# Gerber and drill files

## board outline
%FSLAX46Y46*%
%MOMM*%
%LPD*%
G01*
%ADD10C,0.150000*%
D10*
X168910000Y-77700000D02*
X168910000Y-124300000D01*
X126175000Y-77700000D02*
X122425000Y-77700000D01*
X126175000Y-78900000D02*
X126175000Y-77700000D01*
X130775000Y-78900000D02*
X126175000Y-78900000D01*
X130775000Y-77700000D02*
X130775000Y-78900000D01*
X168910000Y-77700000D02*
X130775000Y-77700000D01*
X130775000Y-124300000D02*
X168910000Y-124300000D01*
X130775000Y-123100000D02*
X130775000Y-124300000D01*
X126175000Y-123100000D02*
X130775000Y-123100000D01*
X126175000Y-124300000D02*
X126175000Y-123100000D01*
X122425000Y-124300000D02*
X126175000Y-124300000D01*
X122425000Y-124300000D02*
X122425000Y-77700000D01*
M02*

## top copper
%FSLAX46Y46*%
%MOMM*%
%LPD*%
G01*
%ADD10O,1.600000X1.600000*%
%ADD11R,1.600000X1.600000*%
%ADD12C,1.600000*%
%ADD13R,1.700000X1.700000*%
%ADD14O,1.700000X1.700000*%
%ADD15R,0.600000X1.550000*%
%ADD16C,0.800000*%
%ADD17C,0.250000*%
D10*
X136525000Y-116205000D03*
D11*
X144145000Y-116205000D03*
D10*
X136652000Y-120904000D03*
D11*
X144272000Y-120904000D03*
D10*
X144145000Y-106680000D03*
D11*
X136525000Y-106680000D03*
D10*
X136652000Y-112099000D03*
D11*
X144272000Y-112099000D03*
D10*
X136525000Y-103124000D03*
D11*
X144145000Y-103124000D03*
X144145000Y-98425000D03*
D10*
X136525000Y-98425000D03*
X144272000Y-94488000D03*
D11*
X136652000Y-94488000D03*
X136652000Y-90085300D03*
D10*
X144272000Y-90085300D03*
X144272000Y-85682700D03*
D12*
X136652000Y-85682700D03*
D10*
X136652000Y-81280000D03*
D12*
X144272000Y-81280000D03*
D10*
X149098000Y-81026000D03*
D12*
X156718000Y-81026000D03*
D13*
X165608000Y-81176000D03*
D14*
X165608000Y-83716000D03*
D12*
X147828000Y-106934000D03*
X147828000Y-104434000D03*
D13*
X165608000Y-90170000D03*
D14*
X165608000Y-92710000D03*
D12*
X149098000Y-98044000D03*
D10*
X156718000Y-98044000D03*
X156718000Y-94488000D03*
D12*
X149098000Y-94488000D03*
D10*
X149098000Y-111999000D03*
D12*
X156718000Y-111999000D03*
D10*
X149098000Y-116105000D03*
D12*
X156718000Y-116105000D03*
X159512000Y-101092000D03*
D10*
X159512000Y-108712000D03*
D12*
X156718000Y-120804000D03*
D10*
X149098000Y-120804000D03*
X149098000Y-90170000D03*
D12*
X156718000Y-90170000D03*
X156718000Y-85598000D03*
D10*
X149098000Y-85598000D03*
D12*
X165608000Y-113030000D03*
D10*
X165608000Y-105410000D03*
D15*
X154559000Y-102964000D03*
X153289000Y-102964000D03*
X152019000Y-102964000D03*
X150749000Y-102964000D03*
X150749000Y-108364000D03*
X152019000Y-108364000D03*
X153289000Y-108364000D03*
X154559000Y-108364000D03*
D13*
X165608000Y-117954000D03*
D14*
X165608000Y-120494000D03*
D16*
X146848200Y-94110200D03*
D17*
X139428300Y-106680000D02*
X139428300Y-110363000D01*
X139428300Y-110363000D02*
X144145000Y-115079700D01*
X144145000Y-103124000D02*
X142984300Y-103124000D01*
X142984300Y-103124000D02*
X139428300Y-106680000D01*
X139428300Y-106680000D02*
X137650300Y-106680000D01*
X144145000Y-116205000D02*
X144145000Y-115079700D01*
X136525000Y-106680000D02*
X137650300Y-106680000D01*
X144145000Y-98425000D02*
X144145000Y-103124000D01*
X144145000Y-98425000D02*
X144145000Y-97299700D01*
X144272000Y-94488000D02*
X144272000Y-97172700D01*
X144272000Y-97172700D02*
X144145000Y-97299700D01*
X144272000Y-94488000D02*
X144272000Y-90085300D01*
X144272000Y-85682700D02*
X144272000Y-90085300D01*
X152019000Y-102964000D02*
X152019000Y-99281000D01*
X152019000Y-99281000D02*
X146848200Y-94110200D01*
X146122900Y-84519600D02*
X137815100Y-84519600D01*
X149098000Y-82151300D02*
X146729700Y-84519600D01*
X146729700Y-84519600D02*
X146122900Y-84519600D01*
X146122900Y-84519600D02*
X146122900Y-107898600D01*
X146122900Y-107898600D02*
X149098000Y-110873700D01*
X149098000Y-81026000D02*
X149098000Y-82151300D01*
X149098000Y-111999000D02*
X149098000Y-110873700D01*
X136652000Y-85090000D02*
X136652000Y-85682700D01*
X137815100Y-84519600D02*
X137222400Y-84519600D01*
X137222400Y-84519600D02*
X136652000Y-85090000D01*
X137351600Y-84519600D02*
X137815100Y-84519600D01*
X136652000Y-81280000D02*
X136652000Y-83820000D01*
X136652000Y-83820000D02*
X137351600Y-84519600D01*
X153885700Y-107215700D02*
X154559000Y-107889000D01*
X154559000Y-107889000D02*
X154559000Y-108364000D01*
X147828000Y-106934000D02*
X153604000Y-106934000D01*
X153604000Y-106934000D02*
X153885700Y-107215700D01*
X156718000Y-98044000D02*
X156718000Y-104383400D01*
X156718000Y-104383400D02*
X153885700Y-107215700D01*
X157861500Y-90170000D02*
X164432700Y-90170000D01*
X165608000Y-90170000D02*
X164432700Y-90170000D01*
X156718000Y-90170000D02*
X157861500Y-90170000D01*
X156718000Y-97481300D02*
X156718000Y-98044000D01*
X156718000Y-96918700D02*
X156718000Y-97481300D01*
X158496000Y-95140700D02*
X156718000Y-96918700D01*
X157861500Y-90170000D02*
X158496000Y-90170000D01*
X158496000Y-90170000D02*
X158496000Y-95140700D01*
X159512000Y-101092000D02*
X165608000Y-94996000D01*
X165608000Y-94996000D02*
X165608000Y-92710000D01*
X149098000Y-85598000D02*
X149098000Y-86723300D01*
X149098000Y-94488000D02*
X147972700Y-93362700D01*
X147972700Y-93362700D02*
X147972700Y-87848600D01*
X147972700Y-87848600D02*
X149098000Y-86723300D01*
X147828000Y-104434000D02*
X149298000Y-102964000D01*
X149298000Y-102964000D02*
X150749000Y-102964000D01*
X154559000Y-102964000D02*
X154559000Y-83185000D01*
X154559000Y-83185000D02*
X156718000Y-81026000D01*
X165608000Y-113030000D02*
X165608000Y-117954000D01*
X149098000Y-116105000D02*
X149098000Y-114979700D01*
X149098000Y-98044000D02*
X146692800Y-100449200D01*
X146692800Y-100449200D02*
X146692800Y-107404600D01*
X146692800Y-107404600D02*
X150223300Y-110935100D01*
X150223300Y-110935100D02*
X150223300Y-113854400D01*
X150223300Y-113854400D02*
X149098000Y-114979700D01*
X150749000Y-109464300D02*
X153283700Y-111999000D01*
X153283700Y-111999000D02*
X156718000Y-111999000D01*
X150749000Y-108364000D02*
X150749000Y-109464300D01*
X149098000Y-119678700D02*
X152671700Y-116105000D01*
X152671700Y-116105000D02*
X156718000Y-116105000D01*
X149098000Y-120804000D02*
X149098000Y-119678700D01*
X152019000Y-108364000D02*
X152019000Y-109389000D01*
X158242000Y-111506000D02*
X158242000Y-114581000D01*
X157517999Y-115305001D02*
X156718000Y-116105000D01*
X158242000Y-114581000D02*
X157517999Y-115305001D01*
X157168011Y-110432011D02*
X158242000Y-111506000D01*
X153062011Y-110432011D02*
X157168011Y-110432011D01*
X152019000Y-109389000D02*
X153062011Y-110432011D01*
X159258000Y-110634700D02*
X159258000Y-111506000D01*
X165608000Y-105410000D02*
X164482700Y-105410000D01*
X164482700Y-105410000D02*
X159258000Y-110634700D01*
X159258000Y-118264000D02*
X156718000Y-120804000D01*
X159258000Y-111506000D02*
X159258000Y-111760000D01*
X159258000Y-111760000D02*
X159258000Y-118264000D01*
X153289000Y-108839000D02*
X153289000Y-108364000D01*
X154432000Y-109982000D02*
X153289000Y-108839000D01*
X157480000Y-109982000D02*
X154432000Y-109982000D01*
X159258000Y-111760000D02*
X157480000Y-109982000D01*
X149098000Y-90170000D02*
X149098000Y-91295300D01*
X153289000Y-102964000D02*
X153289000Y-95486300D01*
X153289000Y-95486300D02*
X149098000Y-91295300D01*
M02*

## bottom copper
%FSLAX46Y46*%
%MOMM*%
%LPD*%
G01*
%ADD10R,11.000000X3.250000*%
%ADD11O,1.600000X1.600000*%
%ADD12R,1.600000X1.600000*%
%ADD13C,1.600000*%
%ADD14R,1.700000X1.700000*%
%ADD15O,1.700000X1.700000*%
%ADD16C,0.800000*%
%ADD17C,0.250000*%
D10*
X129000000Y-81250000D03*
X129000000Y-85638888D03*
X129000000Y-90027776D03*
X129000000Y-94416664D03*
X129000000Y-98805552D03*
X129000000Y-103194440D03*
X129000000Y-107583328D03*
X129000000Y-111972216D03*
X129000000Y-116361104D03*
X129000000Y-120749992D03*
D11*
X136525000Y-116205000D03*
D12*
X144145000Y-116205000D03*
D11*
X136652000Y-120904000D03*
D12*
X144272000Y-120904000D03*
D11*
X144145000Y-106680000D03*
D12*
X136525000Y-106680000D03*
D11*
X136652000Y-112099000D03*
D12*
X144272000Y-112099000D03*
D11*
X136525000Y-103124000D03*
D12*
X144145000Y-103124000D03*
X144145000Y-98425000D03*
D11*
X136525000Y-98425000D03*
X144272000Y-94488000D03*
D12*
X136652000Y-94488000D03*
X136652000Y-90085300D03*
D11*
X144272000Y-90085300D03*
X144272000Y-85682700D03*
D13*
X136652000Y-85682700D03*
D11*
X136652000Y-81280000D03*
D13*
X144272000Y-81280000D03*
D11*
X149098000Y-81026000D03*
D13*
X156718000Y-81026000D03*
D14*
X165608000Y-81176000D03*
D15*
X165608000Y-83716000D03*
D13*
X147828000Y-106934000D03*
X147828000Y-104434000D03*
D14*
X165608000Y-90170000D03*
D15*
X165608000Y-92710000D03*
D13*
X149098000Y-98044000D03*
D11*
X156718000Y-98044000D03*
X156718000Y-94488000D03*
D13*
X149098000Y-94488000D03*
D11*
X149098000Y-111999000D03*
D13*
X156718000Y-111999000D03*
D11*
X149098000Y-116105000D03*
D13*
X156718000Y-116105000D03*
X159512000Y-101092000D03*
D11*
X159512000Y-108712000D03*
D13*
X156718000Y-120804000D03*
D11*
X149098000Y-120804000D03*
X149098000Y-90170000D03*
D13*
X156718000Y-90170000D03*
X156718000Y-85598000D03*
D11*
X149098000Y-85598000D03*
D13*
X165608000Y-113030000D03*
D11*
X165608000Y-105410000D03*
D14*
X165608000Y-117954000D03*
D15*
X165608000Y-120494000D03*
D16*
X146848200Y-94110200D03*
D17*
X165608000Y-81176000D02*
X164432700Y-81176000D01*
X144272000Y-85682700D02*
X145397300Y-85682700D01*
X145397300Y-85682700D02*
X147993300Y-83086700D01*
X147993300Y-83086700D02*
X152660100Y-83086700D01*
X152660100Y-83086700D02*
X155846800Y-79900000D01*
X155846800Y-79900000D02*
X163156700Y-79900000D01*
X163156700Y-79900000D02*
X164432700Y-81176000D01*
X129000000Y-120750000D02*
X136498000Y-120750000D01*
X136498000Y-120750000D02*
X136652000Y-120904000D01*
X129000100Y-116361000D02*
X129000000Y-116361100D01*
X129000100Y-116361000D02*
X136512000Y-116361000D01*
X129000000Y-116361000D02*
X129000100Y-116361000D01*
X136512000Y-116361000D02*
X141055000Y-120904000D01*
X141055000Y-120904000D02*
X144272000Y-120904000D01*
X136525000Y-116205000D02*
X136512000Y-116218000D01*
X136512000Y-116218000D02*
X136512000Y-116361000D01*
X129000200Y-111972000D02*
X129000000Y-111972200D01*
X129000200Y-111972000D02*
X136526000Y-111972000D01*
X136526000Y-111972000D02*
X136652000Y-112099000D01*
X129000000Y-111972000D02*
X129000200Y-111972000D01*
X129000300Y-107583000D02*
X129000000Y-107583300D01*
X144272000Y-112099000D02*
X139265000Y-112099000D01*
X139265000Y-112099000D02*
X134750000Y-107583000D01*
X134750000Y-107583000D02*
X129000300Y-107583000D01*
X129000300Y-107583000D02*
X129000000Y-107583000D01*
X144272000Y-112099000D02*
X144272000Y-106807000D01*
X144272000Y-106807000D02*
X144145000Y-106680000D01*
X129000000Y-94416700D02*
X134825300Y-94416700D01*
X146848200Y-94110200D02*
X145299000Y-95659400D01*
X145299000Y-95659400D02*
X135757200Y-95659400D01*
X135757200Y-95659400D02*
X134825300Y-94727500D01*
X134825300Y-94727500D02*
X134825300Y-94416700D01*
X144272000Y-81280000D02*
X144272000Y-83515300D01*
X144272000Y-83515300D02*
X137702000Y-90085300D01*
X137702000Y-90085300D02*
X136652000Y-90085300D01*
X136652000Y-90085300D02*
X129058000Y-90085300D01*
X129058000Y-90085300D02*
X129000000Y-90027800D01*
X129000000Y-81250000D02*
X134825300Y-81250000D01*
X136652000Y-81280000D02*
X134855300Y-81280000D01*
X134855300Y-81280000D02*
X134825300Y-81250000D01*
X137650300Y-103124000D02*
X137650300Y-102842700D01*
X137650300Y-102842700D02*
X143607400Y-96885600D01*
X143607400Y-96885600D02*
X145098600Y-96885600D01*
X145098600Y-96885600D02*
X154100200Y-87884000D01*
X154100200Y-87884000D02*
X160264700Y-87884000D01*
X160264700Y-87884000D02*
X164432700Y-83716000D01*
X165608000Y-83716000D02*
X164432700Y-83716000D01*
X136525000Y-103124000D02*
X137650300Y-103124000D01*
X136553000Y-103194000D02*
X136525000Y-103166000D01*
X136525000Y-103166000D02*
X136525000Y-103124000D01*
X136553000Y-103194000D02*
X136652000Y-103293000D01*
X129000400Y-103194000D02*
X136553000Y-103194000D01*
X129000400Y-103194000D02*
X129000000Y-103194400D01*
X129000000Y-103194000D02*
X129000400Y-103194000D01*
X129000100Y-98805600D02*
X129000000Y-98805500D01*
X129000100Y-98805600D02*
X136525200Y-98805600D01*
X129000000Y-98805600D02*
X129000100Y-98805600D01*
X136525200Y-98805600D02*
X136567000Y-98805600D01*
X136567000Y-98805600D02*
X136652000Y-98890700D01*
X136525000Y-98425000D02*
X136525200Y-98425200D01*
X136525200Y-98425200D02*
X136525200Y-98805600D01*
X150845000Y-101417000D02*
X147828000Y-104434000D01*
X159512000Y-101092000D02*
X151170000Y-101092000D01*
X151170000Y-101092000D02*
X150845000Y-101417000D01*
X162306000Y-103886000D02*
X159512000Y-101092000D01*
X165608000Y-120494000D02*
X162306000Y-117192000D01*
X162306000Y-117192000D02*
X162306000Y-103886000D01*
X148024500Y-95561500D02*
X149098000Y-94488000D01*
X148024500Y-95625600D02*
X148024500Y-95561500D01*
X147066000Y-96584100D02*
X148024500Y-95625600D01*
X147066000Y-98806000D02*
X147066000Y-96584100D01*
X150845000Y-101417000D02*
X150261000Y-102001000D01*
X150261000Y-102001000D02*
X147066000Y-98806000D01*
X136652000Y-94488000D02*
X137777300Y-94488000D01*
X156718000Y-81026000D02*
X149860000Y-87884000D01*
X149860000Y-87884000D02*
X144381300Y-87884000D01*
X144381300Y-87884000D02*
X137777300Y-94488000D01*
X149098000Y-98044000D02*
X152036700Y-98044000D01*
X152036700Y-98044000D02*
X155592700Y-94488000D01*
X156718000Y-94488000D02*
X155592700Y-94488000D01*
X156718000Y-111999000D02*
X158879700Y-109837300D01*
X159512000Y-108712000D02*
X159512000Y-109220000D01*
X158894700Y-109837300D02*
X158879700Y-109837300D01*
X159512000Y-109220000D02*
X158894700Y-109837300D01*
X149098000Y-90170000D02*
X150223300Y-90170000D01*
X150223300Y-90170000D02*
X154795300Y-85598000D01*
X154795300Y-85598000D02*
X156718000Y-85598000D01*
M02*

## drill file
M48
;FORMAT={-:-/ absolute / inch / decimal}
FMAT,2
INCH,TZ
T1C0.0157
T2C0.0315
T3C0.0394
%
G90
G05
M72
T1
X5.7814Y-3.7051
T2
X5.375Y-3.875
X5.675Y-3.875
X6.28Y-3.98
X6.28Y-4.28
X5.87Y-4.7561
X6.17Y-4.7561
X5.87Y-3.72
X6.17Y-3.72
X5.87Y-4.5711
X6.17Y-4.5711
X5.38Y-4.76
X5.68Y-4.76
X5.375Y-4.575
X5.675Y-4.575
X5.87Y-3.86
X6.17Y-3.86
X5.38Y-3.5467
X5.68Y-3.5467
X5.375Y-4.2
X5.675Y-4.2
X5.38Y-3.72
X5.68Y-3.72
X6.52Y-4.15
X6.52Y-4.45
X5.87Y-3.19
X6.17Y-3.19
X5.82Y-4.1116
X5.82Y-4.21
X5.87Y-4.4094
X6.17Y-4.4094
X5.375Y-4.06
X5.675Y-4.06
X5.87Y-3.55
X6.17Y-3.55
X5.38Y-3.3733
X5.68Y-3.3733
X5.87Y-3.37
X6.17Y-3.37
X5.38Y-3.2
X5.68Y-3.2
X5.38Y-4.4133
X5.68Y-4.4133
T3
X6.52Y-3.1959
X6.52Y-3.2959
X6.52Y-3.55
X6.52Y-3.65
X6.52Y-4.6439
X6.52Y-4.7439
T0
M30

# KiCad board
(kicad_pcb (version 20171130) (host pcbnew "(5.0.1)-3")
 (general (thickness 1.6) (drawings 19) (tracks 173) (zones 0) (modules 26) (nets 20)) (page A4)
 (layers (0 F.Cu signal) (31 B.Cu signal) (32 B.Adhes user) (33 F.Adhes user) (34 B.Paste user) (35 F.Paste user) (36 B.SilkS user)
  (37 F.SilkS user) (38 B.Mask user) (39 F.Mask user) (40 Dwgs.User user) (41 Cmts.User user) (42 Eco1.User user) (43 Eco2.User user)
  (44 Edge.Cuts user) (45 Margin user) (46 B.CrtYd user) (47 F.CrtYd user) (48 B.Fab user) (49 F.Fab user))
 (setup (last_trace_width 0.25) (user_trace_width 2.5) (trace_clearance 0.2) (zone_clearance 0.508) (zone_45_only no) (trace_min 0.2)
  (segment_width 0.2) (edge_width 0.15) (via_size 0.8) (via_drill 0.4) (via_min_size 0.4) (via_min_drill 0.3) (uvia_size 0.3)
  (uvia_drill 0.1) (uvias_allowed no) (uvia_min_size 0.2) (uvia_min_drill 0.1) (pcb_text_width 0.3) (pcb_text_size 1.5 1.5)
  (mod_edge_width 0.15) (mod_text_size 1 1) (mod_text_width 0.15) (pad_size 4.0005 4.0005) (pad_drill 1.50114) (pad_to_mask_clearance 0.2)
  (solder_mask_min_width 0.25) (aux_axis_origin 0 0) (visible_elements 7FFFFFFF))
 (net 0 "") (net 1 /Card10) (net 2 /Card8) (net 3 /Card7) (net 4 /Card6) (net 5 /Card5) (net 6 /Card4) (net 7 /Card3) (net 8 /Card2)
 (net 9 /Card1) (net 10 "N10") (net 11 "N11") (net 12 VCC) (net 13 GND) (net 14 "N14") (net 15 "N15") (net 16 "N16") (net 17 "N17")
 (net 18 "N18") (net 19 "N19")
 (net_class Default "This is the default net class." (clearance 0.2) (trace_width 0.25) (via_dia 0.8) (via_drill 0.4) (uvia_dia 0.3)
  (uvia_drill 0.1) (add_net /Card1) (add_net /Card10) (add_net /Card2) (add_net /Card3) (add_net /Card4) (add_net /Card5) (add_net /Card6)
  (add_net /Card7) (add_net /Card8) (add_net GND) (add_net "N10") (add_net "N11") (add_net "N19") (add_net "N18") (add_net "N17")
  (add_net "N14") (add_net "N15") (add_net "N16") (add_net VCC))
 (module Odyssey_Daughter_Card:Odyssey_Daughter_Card (layer F.Cu) (at 129 101)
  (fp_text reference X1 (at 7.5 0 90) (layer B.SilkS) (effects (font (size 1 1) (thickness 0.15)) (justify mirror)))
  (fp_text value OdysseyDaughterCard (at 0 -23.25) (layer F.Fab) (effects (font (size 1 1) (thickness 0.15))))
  (pad 10 smd rect (at 0 -19.75) (size 11 3.25) (layers B.Cu B.Mask) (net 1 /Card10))
  (pad 9 smd rect (at 0 -15.361112) (size 11 3.25) (layers B.Cu B.Mask))
  (pad 8 smd rect (at 0 -10.972224) (size 11 3.25) (layers B.Cu B.Mask) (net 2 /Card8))
  (pad 7 smd rect (at 0 -6.583336) (size 11 3.25) (layers B.Cu B.Mask) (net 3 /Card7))
  (pad 6 smd rect (at 0 -2.194448) (size 11 3.25) (layers B.Cu B.Mask) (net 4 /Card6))
  (pad 5 smd rect (at 0 2.19444) (size 11 3.25) (layers B.Cu B.Mask) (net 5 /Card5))
  (pad 4 smd rect (at 0 6.583328) (size 11 3.25) (layers B.Cu B.Mask) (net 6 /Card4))
  (pad 3 smd rect (at 0 10.972216) (size 11 3.25) (layers B.Cu B.Mask) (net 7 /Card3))
  (pad 2 smd rect (at 0 15.361104) (size 11 3.25) (layers B.Cu B.Mask) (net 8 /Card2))
  (pad 1 smd rect (at 0 19.749992) (size 11 3.25) (layers B.Cu B.Mask) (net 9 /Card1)))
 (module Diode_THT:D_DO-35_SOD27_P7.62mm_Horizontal (layer F.Cu) (at 144.145 116.205 180)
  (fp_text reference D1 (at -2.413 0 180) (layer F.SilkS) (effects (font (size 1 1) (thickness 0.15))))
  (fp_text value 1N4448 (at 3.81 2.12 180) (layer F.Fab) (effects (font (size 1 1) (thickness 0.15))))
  (pad 2 thru_hole oval (at 7.62 0 180) (size 1.6 1.6) (drill 0.8) (layers *.Cu *.Mask) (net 8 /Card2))
  (pad 1 thru_hole rect (at 0 0 180) (size 1.6 1.6) (drill 0.8) (layers *.Cu *.Mask) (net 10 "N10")))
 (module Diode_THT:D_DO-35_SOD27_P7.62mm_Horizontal (layer F.Cu) (at 144.272 120.904 180)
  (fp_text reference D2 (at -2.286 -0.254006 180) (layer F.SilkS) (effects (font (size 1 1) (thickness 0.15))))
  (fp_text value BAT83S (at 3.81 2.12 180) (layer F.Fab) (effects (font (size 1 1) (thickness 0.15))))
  (pad 2 thru_hole oval (at 7.62 0 180) (size 1.6 1.6) (drill 0.8) (layers *.Cu *.Mask) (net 9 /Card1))
  (pad 1 thru_hole rect (at 0 0 180) (size 1.6 1.6) (drill 0.8) (layers *.Cu *.Mask) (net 8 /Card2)))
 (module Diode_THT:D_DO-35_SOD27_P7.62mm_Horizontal (layer F.Cu) (at 136.525 106.68)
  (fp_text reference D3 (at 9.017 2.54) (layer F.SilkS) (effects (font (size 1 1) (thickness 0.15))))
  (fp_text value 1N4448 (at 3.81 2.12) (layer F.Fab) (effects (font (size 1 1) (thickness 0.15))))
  (pad 2 thru_hole oval (at 7.62 0) (size 1.6 1.6) (drill 0.8) (layers *.Cu *.Mask) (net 6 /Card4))
  (pad 1 thru_hole rect (at 0 0) (size 1.6 1.6) (drill 0.8) (layers *.Cu *.Mask) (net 10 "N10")))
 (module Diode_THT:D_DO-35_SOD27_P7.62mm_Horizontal (layer F.Cu) (at 144.272 112.099 180)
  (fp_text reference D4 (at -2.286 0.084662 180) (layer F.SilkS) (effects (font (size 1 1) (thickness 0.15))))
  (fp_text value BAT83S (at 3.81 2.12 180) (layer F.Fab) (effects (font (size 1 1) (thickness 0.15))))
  (pad 2 thru_hole oval (at 7.62 0 180) (size 1.6 1.6) (drill 0.8) (layers *.Cu *.Mask) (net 7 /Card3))
  (pad 1 thru_hole rect (at 0 0 180) (size 1.6 1.6) (drill 0.8) (layers *.Cu *.Mask) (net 6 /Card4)))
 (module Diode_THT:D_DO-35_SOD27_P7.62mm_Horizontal (layer F.Cu) (at 144.145 103.124 180)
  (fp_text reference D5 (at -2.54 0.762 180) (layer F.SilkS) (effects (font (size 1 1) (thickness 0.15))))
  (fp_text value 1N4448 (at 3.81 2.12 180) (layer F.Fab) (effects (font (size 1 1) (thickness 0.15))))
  (pad 2 thru_hole oval (at 7.62 0 180) (size 1.6 1.6) (drill 0.8) (layers *.Cu *.Mask) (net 5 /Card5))
  (pad 1 thru_hole rect (at 0 0 180) (size 1.6 1.6) (drill 0.8) (layers *.Cu *.Mask) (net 10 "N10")))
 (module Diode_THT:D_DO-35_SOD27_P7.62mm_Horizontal (layer F.Cu) (at 144.145 98.425 180)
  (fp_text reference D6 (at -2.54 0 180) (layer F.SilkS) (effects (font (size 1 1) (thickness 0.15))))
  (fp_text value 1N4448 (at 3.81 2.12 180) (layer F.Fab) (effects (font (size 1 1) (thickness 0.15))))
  (pad 1 thru_hole rect (at 0 0 180) (size 1.6 1.6) (drill 0.8) (layers *.Cu *.Mask) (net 10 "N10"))
  (pad 2 thru_hole oval (at 7.62 0 180) (size 1.6 1.6) (drill 0.8) (layers *.Cu *.Mask) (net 4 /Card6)))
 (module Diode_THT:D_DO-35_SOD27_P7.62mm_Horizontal (layer F.Cu) (at 136.652 94.488)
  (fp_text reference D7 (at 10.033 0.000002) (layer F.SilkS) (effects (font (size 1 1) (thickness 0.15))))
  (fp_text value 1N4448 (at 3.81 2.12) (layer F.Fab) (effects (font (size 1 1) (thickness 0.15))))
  (pad 2 thru_hole oval (at 7.62 0) (size 1.6 1.6) (drill 0.8) (layers *.Cu *.Mask) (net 10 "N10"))
  (pad 1 thru_hole rect (at 0 0) (size 1.6 1.6) (drill 0.8) (layers *.Cu *.Mask) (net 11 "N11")))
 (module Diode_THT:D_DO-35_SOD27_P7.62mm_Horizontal (layer F.Cu) (at 136.652 90.0853)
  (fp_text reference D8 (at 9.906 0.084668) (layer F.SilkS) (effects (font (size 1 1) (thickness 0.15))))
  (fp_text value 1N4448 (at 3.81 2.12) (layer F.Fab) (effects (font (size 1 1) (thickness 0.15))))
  (pad 1 thru_hole rect (at 0 0) (size 1.6 1.6) (drill 0.8) (layers *.Cu *.Mask) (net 2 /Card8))
  (pad 2 thru_hole oval (at 7.62 0) (size 1.6 1.6) (drill 0.8) (layers *.Cu *.Mask) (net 10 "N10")))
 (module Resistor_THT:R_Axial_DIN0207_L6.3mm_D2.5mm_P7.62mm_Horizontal (layer F.Cu) (at 136.652 85.6827)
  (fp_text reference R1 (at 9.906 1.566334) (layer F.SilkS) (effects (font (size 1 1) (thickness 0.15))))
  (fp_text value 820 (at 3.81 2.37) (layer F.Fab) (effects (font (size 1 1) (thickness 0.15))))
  (pad 2 thru_hole oval (at 7.62 0) (size 1.6 1.6) (drill 0.8) (layers *.Cu *.Mask) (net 10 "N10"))
  (pad 1 thru_hole circle (at 0 0) (size 1.6 1.6) (drill 0.8) (layers *.Cu *.Mask) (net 1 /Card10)))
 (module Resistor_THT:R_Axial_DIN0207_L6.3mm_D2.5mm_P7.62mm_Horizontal (layer F.Cu) (at 144.272 81.28 180)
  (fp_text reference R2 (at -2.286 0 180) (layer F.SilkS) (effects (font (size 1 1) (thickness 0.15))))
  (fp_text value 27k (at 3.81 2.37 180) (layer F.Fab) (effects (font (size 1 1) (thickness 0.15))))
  (pad 2 thru_hole oval (at 7.62 0 180) (size 1.6 1.6) (drill 0.8) (layers *.Cu *.Mask) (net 1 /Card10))
  (pad 1 thru_hole circle (at 0 0 180) (size 1.6 1.6) (drill 0.8) (layers *.Cu *.Mask) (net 2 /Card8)))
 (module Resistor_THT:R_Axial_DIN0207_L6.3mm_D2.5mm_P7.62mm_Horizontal (layer F.Cu) (at 156.718 81.026 180)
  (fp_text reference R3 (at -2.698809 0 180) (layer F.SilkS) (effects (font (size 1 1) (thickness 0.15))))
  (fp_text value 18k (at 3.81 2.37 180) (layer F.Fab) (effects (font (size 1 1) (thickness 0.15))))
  (pad 2 thru_hole oval (at 7.62 0 180) (size 1.6 1.6) (drill 0.8) (layers *.Cu *.Mask) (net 1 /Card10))
  (pad 1 thru_hole circle (at 0 0 180) (size 1.6 1.6) (drill 0.8) (layers *.Cu *.Mask) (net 11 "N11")))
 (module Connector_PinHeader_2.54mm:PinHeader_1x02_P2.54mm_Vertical (layer F.Cu) (at 165.608 81.176)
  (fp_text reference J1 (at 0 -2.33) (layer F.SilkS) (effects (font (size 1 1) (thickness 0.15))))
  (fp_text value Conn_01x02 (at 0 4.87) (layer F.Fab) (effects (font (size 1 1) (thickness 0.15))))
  (pad 1 thru_hole rect (at 0 0) (size 1.7 1.7) (drill 1) (layers *.Cu *.Mask) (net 10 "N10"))
  (pad 2 thru_hole oval (at 0 2.54) (size 1.7 1.7) (drill 1) (layers *.Cu *.Mask) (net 5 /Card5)))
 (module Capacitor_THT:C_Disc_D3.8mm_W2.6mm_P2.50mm (layer F.Cu) (at 147.828 106.934 90)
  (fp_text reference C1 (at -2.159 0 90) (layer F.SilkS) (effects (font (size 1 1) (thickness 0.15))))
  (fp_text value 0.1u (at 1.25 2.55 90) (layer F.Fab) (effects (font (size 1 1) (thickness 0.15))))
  (pad 1 thru_hole circle (at 0 0 90) (size 1.6 1.6) (drill 0.8) (layers *.Cu *.Mask) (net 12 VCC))
  (pad 2 thru_hole circle (at 2.5 0 90) (size 1.6 1.6) (drill 0.8) (layers *.Cu *.Mask) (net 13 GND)))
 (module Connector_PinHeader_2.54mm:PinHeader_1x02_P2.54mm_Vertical (layer F.Cu) (at 165.608 90.17)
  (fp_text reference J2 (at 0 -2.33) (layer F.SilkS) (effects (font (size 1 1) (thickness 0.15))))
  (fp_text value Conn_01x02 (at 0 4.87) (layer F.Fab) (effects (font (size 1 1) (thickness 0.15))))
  (pad 1 thru_hole rect (at 0 0) (size 1.7 1.7) (drill 1) (layers *.Cu *.Mask) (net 12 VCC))
  (pad 2 thru_hole oval (at 0 2.54) (size 1.7 1.7) (drill 1) (layers *.Cu *.Mask) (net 13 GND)))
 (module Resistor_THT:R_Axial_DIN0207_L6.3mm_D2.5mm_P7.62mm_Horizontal (layer F.Cu) (at 149.098 98.044)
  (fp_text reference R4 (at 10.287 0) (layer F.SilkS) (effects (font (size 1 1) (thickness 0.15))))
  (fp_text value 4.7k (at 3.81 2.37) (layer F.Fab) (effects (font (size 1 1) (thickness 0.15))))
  (pad 1 thru_hole circle (at 0 0) (size 1.6 1.6) (drill 0.8) (layers *.Cu *.Mask) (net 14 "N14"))
  (pad 2 thru_hole oval (at 7.62 0) (size 1.6 1.6) (drill 0.8) (layers *.Cu *.Mask) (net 12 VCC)))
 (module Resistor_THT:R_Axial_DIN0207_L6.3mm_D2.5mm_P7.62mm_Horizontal (layer F.Cu) (at 149.098 94.488)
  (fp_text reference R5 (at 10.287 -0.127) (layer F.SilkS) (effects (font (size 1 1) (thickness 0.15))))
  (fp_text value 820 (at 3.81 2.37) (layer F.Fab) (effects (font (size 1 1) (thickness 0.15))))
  (pad 2 thru_hole oval (at 7.62 0) (size 1.6 1.6) (drill 0.8) (layers *.Cu *.Mask) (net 14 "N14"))
  (pad 1 thru_hole circle (at 0 0) (size 1.6 1.6) (drill 0.8) (layers *.Cu *.Mask) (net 13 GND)))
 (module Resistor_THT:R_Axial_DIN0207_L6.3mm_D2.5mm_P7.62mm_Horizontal (layer F.Cu) (at 156.718 111.999 180)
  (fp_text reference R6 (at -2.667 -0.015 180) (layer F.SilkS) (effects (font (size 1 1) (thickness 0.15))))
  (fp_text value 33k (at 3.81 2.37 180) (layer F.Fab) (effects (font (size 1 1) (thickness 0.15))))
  (pad 2 thru_hole oval (at 7.62 0 180) (size 1.6 1.6) (drill 0.8) (layers *.Cu *.Mask) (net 1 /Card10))
  (pad 1 thru_hole circle (at 0 0 180) (size 1.6 1.6) (drill 0.8) (layers *.Cu *.Mask) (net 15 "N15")))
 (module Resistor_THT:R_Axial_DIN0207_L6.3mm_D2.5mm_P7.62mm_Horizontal (layer F.Cu) (at 156.718 116.105 180)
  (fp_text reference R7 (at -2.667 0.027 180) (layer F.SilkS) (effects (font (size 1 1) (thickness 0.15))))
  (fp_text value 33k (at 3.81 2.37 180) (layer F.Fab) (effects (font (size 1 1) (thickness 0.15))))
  (pad 2 thru_hole oval (at 7.62 0 180) (size 1.6 1.6) (drill 0.8) (layers *.Cu *.Mask) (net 14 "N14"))
  (pad 1 thru_hole circle (at 0 0 180) (size 1.6 1.6) (drill 0.8) (layers *.Cu *.Mask) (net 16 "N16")))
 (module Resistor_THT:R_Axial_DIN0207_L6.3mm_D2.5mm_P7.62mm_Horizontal (layer F.Cu) (at 159.512 101.092 270)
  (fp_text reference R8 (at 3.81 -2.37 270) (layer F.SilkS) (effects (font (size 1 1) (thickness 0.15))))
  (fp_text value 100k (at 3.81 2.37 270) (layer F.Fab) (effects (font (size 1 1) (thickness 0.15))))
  (pad 1 thru_hole circle (at 0 0 270) (size 1.6 1.6) (drill 0.8) (layers *.Cu *.Mask) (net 13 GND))
  (pad 2 thru_hole oval (at 7.62 0 270) (size 1.6 1.6) (drill 0.8) (layers *.Cu *.Mask) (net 15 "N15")))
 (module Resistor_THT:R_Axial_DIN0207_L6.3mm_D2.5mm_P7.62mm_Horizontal (layer F.Cu) (at 156.718 120.804 180)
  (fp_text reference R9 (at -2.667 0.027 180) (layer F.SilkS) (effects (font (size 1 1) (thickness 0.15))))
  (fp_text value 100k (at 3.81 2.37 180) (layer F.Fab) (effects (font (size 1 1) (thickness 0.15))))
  (pad 1 thru_hole circle (at 0 0 180) (size 1.6 1.6) (drill 0.8) (layers *.Cu *.Mask) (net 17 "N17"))
  (pad 2 thru_hole oval (at 7.62 0 180) (size 1.6 1.6) (drill 0.8) (layers *.Cu *.Mask) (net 16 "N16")))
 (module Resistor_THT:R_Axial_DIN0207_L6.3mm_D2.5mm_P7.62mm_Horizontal (layer F.Cu) (at 156.718 90.17 180)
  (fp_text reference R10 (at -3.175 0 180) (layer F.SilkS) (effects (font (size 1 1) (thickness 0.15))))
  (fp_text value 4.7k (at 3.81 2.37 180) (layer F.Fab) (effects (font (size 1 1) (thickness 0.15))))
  (pad 2 thru_hole oval (at 7.62 0 180) (size 1.6 1.6) (drill 0.8) (layers *.Cu *.Mask) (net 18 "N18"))
  (pad 1 thru_hole circle (at 0 0 180) (size 1.6 1.6) (drill 0.8) (layers *.Cu *.Mask) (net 12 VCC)))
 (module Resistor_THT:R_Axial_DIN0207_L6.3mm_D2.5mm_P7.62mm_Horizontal (layer F.Cu) (at 156.718 85.598 180)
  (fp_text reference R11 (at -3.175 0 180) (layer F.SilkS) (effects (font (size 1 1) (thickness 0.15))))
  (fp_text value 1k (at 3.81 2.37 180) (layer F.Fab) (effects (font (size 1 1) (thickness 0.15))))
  (pad 1 thru_hole circle (at 0 0 180) (size 1.6 1.6) (drill 0.8) (layers *.Cu *.Mask) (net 18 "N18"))
  (pad 2 thru_hole oval (at 7.62 0 180) (size 1.6 1.6) (drill 0.8) (layers *.Cu *.Mask) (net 13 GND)))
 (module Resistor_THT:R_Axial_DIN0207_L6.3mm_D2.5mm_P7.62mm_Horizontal (layer F.Cu) (at 165.608 113.03 90)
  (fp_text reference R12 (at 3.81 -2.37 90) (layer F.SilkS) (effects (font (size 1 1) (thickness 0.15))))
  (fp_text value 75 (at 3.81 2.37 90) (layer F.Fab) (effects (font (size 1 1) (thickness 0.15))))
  (pad 1 thru_hole circle (at 0 0 90) (size 1.6 1.6) (drill 0.8) (layers *.Cu *.Mask) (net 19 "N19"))
  (pad 2 thru_hole oval (at 7.62 0 90) (size 1.6 1.6) (drill 0.8) (layers *.Cu *.Mask) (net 17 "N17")))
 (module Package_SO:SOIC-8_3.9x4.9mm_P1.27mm (layer F.Cu) (at 152.654 105.664 270)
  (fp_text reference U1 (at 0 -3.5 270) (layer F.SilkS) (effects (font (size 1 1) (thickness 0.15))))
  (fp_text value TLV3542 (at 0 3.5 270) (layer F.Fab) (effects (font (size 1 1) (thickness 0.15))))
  (pad 1 smd rect (at -2.7 -1.905 270) (size 1.55 0.6) (layers F.Cu F.Paste F.Mask) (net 11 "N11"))
  (pad 2 smd rect (at -2.7 -0.635 270) (size 1.55 0.6) (layers F.Cu F.Paste F.Mask) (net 18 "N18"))
  (pad 3 smd rect (at -2.7 0.635 270) (size 1.55 0.6) (layers F.Cu F.Paste F.Mask) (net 3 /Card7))
  (pad 4 smd rect (at -2.7 1.905 270) (size 1.55 0.6) (layers F.Cu F.Paste F.Mask) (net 13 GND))
  (pad 5 smd rect (at 2.7 1.905 270) (size 1.55 0.6) (layers F.Cu F.Paste F.Mask) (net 15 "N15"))
  (pad 6 smd rect (at 2.7 0.635 270) (size 1.55 0.6) (layers F.Cu F.Paste F.Mask) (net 16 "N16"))
  (pad 7 smd rect (at 2.7 -0.635 270) (size 1.55 0.6) (layers F.Cu F.Paste F.Mask) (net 17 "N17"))
  (pad 8 smd rect (at 2.7 -1.905 270) (size 1.55 0.6) (layers F.Cu F.Paste F.Mask) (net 12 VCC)))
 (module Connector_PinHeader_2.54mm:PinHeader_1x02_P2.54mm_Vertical (layer F.Cu) (at 165.608 117.954)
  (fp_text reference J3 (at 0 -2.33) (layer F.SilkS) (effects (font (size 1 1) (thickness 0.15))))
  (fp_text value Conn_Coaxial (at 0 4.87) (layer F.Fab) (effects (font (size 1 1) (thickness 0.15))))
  (pad 1 thru_hole rect (at 0 0) (size 1.7 1.7) (drill 1) (layers *.Cu *.Mask) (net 19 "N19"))
  (pad 2 thru_hole oval (at 0 2.54) (size 1.7 1.7) (drill 1) (layers *.Cu *.Mask) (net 13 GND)))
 (gr_line (start 168.91 77.7) (end 168.91 124.3) (layer Edge.Cuts) (width 0.15))
 (gr_line (start 126.175 77.7) (end 122.425 77.7) (layer Edge.Cuts) (width 0.15))
 (gr_line (start 126.175 78.9) (end 126.175 77.7) (layer Edge.Cuts) (width 0.15))
 (gr_line (start 130.775 78.9) (end 126.175 78.9) (layer Edge.Cuts) (width 0.15))
 (gr_line (start 130.775 77.7) (end 130.775 78.9) (layer Edge.Cuts) (width 0.15))
 (gr_line (start 168.91 77.7) (end 130.775 77.7) (layer Edge.Cuts) (width 0.15))
 (gr_line (start 130.775 124.3) (end 168.91 124.3) (layer Edge.Cuts) (width 0.15))
 (gr_line (start 130.775 123.1) (end 130.775 124.3) (layer Edge.Cuts) (width 0.15))
 (gr_line (start 126.175 123.1) (end 130.775 123.1) (layer Edge.Cuts) (width 0.15))
 (gr_line (start 126.175 124.3) (end 126.175 123.1) (layer Edge.Cuts) (width 0.15))
 (gr_line (start 122.425 124.3) (end 126.175 124.3) (layer Edge.Cuts) (width 0.15))
 (gr_line (start 122.425 124.3) (end 122.425 77.7) (layer Edge.Cuts) (width 0.15))
 (segment (start 139.4283 106.68) (end 139.4283 110.363) (width 0.25) (layer F.Cu) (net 10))
 (segment (start 139.4283 110.363) (end 144.145 115.0797) (width 0.25) (layer F.Cu) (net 10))
 (segment (start 144.145 103.124) (end 142.9843 103.124) (width 0.25) (layer F.Cu) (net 10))
 (segment (start 142.9843 103.124) (end 139.4283 106.68) (width 0.25) (layer F.Cu) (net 10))
 (segment (start 139.4283 106.68) (end 137.6503 106.68) (width 0.25) (layer F.Cu) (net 10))
 (segment (start 144.145 116.205) (end 144.145 115.0797) (width 0.25) (layer F.Cu) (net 10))
 (segment (start 136.525 106.68) (end 137.6503 106.68) (width 0.25) (layer F.Cu) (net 10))
 (segment (start 144.145 98.425) (end 144.145 103.124) (width 0.25) (layer F.Cu) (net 10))
 (segment (start 165.608 81.176) (end 164.4327 81.176) (width 0.25) (layer B.Cu) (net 10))
 (segment (start 144.272 85.6827) (end 145.3973 85.6827) (width 0.25) (layer B.Cu) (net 10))
 (segment (start 145.3973 85.6827) (end 147.9933 83.0867) (width 0.25) (layer B.Cu) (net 10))
 (segment (start 147.9933 83.0867) (end 152.6601 83.0867) (width 0.25) (layer B.Cu) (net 10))
 (segment (start 152.6601 83.0867) (end 155.8468 79.9) (width 0.25) (layer B.Cu) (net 10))
 (segment (start 155.8468 79.9) (end 163.1567 79.9) (width 0.25) (layer B.Cu) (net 10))
 (segment (start 163.1567 79.9) (end 164.4327 81.176) (width 0.25) (layer B.Cu) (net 10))
 (segment (start 144.145 98.425) (end 144.145 97.2997) (width 0.25) (layer F.Cu) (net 10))
 (segment (start 144.272 94.488) (end 144.272 97.1727) (width 0.25) (layer F.Cu) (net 10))
 (segment (start 144.272 97.1727) (end 144.145 97.2997) (width 0.25) (layer F.Cu) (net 10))
 (segment (start 144.272 94.488) (end 144.272 90.0853) (width 0.25) (layer F.Cu) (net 10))
 (segment (start 144.272 85.6827) (end 144.272 90.0853) (width 0.25) (layer F.Cu) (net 10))
 (segment (start 129 120.75) (end 136.498 120.75) (width 0.25) (layer B.Cu) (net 9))
 (segment (start 136.498 120.75) (end 136.652 120.904) (width 0.25) (layer B.Cu) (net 9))
 (segment (start 129.0001 116.361) (end 129 116.3611) (width 0.25) (layer B.Cu) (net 8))
 (segment (start 129.0001 116.361) (end 136.512 116.361) (width 0.25) (layer B.Cu) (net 8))
 (segment (start 129 116.361) (end 129.0001 116.361) (width 0.25) (layer B.Cu) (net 8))
 (segment (start 136.512 116.361) (end 141.055 120.904) (width 0.25) (layer B.Cu) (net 8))
 (segment (start 141.055 120.904) (end 144.272 120.904) (width 0.25) (layer B.Cu) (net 8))
 (segment (start 136.525 116.205) (end 136.512 116.218) (width 0.25) (layer B.Cu) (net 8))
 (segment (start 136.512 116.218) (end 136.512 116.361) (width 0.25) (layer B.Cu) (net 8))
 (segment (start 129.0002 111.972) (end 129 111.9722) (width 0.25) (layer B.Cu) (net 7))
 (segment (start 129.0002 111.972) (end 136.526 111.972) (width 0.25) (layer B.Cu) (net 7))
 (segment (start 136.526 111.972) (end 136.652 112.099) (width 0.25) (layer B.Cu) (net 7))
 (segment (start 129 111.972) (end 129.0002 111.972) (width 0.25) (layer B.Cu) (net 7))
 (segment (start 129.0003 107.583) (end 129 107.5833) (width 0.25) (layer B.Cu) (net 6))
 (segment (start 144.272 112.099) (end 139.265 112.099) (width 0.25) (layer B.Cu) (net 6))
 (segment (start 139.265 112.099) (end 134.75 107.583) (width 0.25) (layer B.Cu) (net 6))
 (segment (start 134.75 107.583) (end 129.0003 107.583) (width 0.25) (layer B.Cu) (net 6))
 (segment (start 129.0003 107.583) (end 129 107.583) (width 0.25) (layer B.Cu) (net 6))
 (segment (start 144.272 112.099) (end 144.272 106.807) (width 0.25) (layer B.Cu) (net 6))
 (segment (start 144.272 106.807) (end 144.145 106.68) (width 0.25) (layer B.Cu) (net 6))
 (segment (start 129 94.4167) (end 134.8253 94.4167) (width 0.25) (layer B.Cu) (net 3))
 (segment (start 146.8482 94.1102) (end 145.299 95.6594) (width 0.25) (layer B.Cu) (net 3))
 (segment (start 145.299 95.6594) (end 135.7572 95.6594) (width 0.25) (layer B.Cu) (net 3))
 (segment (start 135.7572 95.6594) (end 134.8253 94.7275) (width 0.25) (layer B.Cu) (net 3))
 (segment (start 134.8253 94.7275) (end 134.8253 94.4167) (width 0.25) (layer B.Cu) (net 3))
 (segment (start 152.019 102.964) (end 152.019 99.281) (width 0.25) (layer F.Cu) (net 3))
 (segment (start 152.019 99.281) (end 146.8482 94.1102) (width 0.25) (layer F.Cu) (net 3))
 (via (at 146.8482 94.1102) (size 0.8) (layers F.Cu B.Cu) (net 3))
 (segment (start 144.272 81.28) (end 144.272 83.5153) (width 0.25) (layer B.Cu) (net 2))
 (segment (start 144.272 83.5153) (end 137.702 90.0853) (width 0.25) (layer B.Cu) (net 2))
 (segment (start 137.702 90.0853) (end 136.652 90.0853) (width 0.25) (layer B.Cu) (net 2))
 (segment (start 136.652 90.0853) (end 129.058 90.0853) (width 0.25) (layer B.Cu) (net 2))
 (segment (start 129.058 90.0853) (end 129 90.0278) (width 0.25) (layer B.Cu) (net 2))
 (segment (start 146.1229 84.5196) (end 137.8151 84.5196) (width 0.25) (layer F.Cu) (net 1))
 (segment (start 149.098 82.1513) (end 146.7297 84.5196) (width 0.25) (layer F.Cu) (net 1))
 (segment (start 146.7297 84.5196) (end 146.1229 84.5196) (width 0.25) (layer F.Cu) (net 1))
 (segment (start 146.1229 84.5196) (end 146.1229 107.8986) (width 0.25) (layer F.Cu) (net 1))
 (segment (start 146.1229 107.8986) (end 149.098 110.8737) (width 0.25) (layer F.Cu) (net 1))
 (segment (start 129 81.25) (end 134.8253 81.25) (width 0.25) (layer B.Cu) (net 1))
 (segment (start 136.652 81.28) (end 134.8553 81.28) (width 0.25) (layer B.Cu) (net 1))
 (segment (start 134.8553 81.28) (end 134.8253 81.25) (width 0.25) (layer B.Cu) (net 1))
 (segment (start 149.098 81.026) (end 149.098 82.1513) (width 0.25) (layer F.Cu) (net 1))
 (segment (start 149.098 111.999) (end 149.098 110.8737) (width 0.25) (layer F.Cu) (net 1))
 (segment (start 136.652 85.09) (end 136.652 85.6827) (width 0.25) (layer F.Cu) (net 1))
 (segment (start 137.8151 84.5196) (end 137.2224 84.5196) (width 0.25) (layer F.Cu) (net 1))
 (segment (start 137.2224 84.5196) (end 136.652 85.09) (width 0.25) (layer F.Cu) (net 1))
 (segment (start 137.3516 84.5196) (end 137.8151 84.5196) (width 0.25) (layer F.Cu) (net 1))
 (segment (start 136.652 81.28) (end 136.652 83.82) (width 0.25) (layer F.Cu) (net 1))
 (segment (start 136.652 83.82) (end 137.3516 84.5196) (width 0.25) (layer F.Cu) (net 1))
 (segment (start 137.6503 103.124) (end 137.6503 102.8427) (width 0.25) (layer B.Cu) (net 5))
 (segment (start 137.6503 102.8427) (end 143.6074 96.8856) (width 0.25) (layer B.Cu) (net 5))
 (segment (start 143.6074 96.8856) (end 145.0986 96.8856) (width 0.25) (layer B.Cu) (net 5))
 (segment (start 145.0986 96.8856) (end 154.1002 87.884) (width 0.25) (layer B.Cu) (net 5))
 (segment (start 154.1002 87.884) (end 160.2647 87.884) (width 0.25) (layer B.Cu) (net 5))
 (segment (start 160.2647 87.884) (end 164.4327 83.716) (width 0.25) (layer B.Cu) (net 5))
 (segment (start 165.608 83.716) (end 164.4327 83.716) (width 0.25) (layer B.Cu) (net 5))
 (segment (start 136.525 103.124) (end 137.6503 103.124) (width 0.25) (layer B.Cu) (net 5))
 (segment (start 136.553 103.194) (end 136.525 103.166) (width 0.25) (layer B.Cu) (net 5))
 (segment (start 136.525 103.166) (end 136.525 103.124) (width 0.25) (layer B.Cu) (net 5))
 (segment (start 136.553 103.194) (end 136.652 103.293) (width 0.25) (layer B.Cu) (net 5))
 (segment (start 129.0004 103.194) (end 136.553 103.194) (width 0.25) (layer B.Cu) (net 5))
 (segment (start 129.0004 103.194) (end 129 103.1944) (width 0.25) (layer B.Cu) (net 5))
 (segment (start 129 103.194) (end 129.0004 103.194) (width 0.25) (layer B.Cu) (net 5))
 (segment (start 129.0001 98.8056) (end 129 98.8055) (width 0.25) (layer B.Cu) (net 4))
 (segment (start 129.0001 98.8056) (end 136.5252 98.8056) (width 0.25) (layer B.Cu) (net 4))
 (segment (start 129 98.8056) (end 129.0001 98.8056) (width 0.25) (layer B.Cu) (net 4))
 (segment (start 136.5252 98.8056) (end 136.567 98.8056) (width 0.25) (layer B.Cu) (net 4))
 (segment (start 136.567 98.8056) (end 136.652 98.8907) (width 0.25) (layer B.Cu) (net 4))
 (segment (start 136.525 98.425) (end 136.5252 98.4252) (width 0.25) (layer B.Cu) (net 4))
 (segment (start 136.5252 98.4252) (end 136.5252 98.8056) (width 0.25) (layer B.Cu) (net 4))
 (segment (start 153.8857 107.2157) (end 154.559 107.889) (width 0.25) (layer F.Cu) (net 12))
 (segment (start 154.559 107.889) (end 154.559 108.364) (width 0.25) (layer F.Cu) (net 12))
 (segment (start 147.828 106.934) (end 153.604 106.934) (width 0.25) (layer F.Cu) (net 12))
 (segment (start 153.604 106.934) (end 153.8857 107.2157) (width 0.25) (layer F.Cu) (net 12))
 (segment (start 156.718 98.044) (end 156.718 104.3834) (width 0.25) (layer F.Cu) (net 12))
 (segment (start 156.718 104.3834) (end 153.8857 107.2157) (width 0.25) (layer F.Cu) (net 12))
 (segment (start 157.8615 90.17) (end 164.4327 90.17) (width 0.25) (layer F.Cu) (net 12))
 (segment (start 165.608 90.17) (end 164.4327 90.17) (width 0.25) (layer F.Cu) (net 12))
 (segment (start 156.718 90.17) (end 157.8615 90.17) (width 0.25) (layer F.Cu) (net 12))
 (segment (start 156.718 97.4813) (end 156.718 98.044) (width 0.25) (layer F.Cu) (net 12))
 (segment (start 156.718 96.9187) (end 156.718 97.4813) (width 0.25) (layer F.Cu) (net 12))
 (segment (start 158.496 95.1407) (end 156.718 96.9187) (width 0.25) (layer F.Cu) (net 12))
 (segment (start 157.8615 90.17) (end 158.496 90.17) (width 0.25) (layer F.Cu) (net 12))
 (segment (start 158.496 90.17) (end 158.496 95.1407) (width 0.25) (layer F.Cu) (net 12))
 (segment (start 150.845 101.417) (end 147.828 104.434) (width 0.25) (layer B.Cu) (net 13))
 (segment (start 159.512 101.092) (end 151.17 101.092) (width 0.25) (layer B.Cu) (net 13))
 (segment (start 151.17 101.092) (end 150.845 101.417) (width 0.25) (layer B.Cu) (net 13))
 (segment (start 159.512 101.092) (end 165.608 94.996) (width 0.25) (layer F.Cu) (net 13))
 (segment (start 165.608 94.996) (end 165.608 92.71) (width 0.25) (layer F.Cu) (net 13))
 (segment (start 149.098 85.598) (end 149.098 86.7233) (width 0.25) (layer F.Cu) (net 13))
 (segment (start 149.098 94.488) (end 147.9727 93.3627) (width 0.25) (layer F.Cu) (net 13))
 (segment (start 147.9727 93.3627) (end 147.9727 87.8486) (width 0.25) (layer F.Cu) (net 13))
 (segment (start 147.9727 87.8486) (end 149.098 86.7233) (width 0.25) (layer F.Cu) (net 13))
 (segment (start 147.828 104.434) (end 149.298 102.964) (width 0.25) (layer F.Cu) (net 13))
 (segment (start 149.298 102.964) (end 150.749 102.964) (width 0.25) (layer F.Cu) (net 13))
 (segment (start 162.306 103.886) (end 159.512 101.092) (width 0.25) (layer B.Cu) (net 13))
 (segment (start 165.608 120.494) (end 162.306 117.192) (width 0.25) (layer B.Cu) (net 13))
 (segment (start 162.306 117.192) (end 162.306 103.886) (width 0.25) (layer B.Cu) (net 13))
 (segment (start 148.0245 95.5615) (end 149.098 94.488) (width 0.25) (layer B.Cu) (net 13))
 (segment (start 148.0245 95.6256) (end 148.0245 95.5615) (width 0.25) (layer B.Cu) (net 13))
 (segment (start 147.066 96.5841) (end 148.0245 95.6256) (width 0.25) (layer B.Cu) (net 13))
 (segment (start 147.066 98.806) (end 147.066 96.5841) (width 0.25) (layer B.Cu) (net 13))
 (segment (start 150.845 101.417) (end 150.261 102.001) (width 0.25) (layer B.Cu) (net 13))
 (segment (start 150.261 102.001) (end 147.066 98.806) (width 0.25) (layer B.Cu) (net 13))
 (segment (start 154.559 102.964) (end 154.559 83.185) (width 0.25) (layer F.Cu) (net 11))
 (segment (start 154.559 83.185) (end 156.718 81.026) (width 0.25) (layer F.Cu) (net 11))
 (segment (start 136.652 94.488) (end 137.7773 94.488) (width 0.25) (layer B.Cu) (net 11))
 (segment (start 156.718 81.026) (end 149.86 87.884) (width 0.25) (layer B.Cu) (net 11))
 (segment (start 149.86 87.884) (end 144.3813 87.884) (width 0.25) (layer B.Cu) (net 11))
 (segment (start 144.3813 87.884) (end 137.7773 94.488) (width 0.25) (layer B.Cu) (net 11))
 (segment (start 165.608 113.03) (end 165.608 117.954) (width 0.25) (layer F.Cu) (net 19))
 (segment (start 149.098 98.044) (end 152.0367 98.044) (width 0.25) (layer B.Cu) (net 14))
 (segment (start 152.0367 98.044) (end 155.5927 94.488) (width 0.25) (layer B.Cu) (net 14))
 (segment (start 149.098 116.105) (end 149.098 114.9797) (width 0.25) (layer F.Cu) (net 14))
 (segment (start 149.098 98.044) (end 146.6928 100.4492) (width 0.25) (layer F.Cu) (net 14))
 (segment (start 146.6928 100.4492) (end 146.6928 107.4046) (width 0.25) (layer F.Cu) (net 14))
 (segment (start 146.6928 107.4046) (end 150.2233 110.9351) (width 0.25) (layer F.Cu) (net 14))
 (segment (start 150.2233 110.9351) (end 150.2233 113.8544) (width 0.25) (layer F.Cu) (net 14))
 (segment (start 150.2233 113.8544) (end 149.098 114.9797) (width 0.25) (layer F.Cu) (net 14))
 (segment (start 156.718 94.488) (end 155.5927 94.488) (width 0.25) (layer B.Cu) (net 14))
 (segment (start 156.718 111.999) (end 158.8797 109.8373) (width 0.25) (layer B.Cu) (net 15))
 (segment (start 150.749 109.4643) (end 153.2837 111.999) (width 0.25) (layer F.Cu) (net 15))
 (segment (start 153.2837 111.999) (end 156.718 111.999) (width 0.25) (layer F.Cu) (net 15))
 (segment (start 150.749 108.364) (end 150.749 109.4643) (width 0.25) (layer F.Cu) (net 15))
 (segment (start 159.512 108.712) (end 159.512 109.22) (width 0.25) (layer B.Cu) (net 15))
 (segment (start 158.8947 109.8373) (end 158.8797 109.8373) (width 0.25) (layer B.Cu) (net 15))
 (segment (start 159.512 109.22) (end 158.8947 109.8373) (width 0.25) (layer B.Cu) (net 15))
 (segment (start 149.098 119.6787) (end 152.6717 116.105) (width 0.25) (layer F.Cu) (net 16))
 (segment (start 152.6717 116.105) (end 156.718 116.105) (width 0.25) (layer F.Cu) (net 16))
 (segment (start 149.098 120.804) (end 149.098 119.6787) (width 0.25) (layer F.Cu) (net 16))
 (segment (start 152.019 108.364) (end 152.019 109.389) (width 0.25) (layer F.Cu) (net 16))
 (segment (start 158.242 111.506) (end 158.242 114.581) (width 0.25) (layer F.Cu) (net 16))
 (segment (start 157.517999 115.305001) (end 156.718 116.105) (width 0.25) (layer F.Cu) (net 16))
 (segment (start 158.242 114.581) (end 157.517999 115.305001) (width 0.25) (layer F.Cu) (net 16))
 (segment (start 157.168011 110.432011) (end 158.242 111.506) (width 0.25) (layer F.Cu) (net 16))
 (segment (start 153.062011 110.432011) (end 157.168011 110.432011) (width 0.25) (layer F.Cu) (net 16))
 (segment (start 152.019 109.389) (end 153.062011 110.432011) (width 0.25) (layer F.Cu) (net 16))
 (segment (start 159.258 110.6347) (end 159.258 111.506) (width 0.25) (layer F.Cu) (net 17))
 (segment (start 165.608 105.41) (end 164.4827 105.41) (width 0.25) (layer F.Cu) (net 17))
 (segment (start 164.4827 105.41) (end 159.258 110.6347) (width 0.25) (layer F.Cu) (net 17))
 (segment (start 159.258 118.264) (end 156.718 120.804) (width 0.25) (layer F.Cu) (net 17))
 (segment (start 159.258 111.506) (end 159.258 111.76) (width 0.25) (layer F.Cu) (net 17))
 (segment (start 159.258 111.76) (end 159.258 118.264) (width 0.25) (layer F.Cu) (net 17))
 (segment (start 153.289 108.839) (end 153.289 108.364) (width 0.25) (layer F.Cu) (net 17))
 (segment (start 154.432 109.982) (end 153.289 108.839) (width 0.25) (layer F.Cu) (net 17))
 (segment (start 157.48 109.982) (end 154.432 109.982) (width 0.25) (layer F.Cu) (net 17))
 (segment (start 159.258 111.76) (end 157.48 109.982) (width 0.25) (layer F.Cu) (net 17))
 (segment (start 149.098 90.17) (end 150.2233 90.17) (width 0.25) (layer B.Cu) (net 18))
 (segment (start 150.2233 90.17) (end 154.7953 85.598) (width 0.25) (layer B.Cu) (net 18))
 (segment (start 154.7953 85.598) (end 156.718 85.598) (width 0.25) (layer B.Cu) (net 18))
 (segment (start 149.098 90.17) (end 149.098 91.2953) (width 0.25) (layer F.Cu) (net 18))
 (segment (start 153.289 102.964) (end 153.289 95.4863) (width 0.25) (layer F.Cu) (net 18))
 (segment (start 153.289 95.4863) (end 149.098 91.2953) (width 0.25) (layer F.Cu) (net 18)))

